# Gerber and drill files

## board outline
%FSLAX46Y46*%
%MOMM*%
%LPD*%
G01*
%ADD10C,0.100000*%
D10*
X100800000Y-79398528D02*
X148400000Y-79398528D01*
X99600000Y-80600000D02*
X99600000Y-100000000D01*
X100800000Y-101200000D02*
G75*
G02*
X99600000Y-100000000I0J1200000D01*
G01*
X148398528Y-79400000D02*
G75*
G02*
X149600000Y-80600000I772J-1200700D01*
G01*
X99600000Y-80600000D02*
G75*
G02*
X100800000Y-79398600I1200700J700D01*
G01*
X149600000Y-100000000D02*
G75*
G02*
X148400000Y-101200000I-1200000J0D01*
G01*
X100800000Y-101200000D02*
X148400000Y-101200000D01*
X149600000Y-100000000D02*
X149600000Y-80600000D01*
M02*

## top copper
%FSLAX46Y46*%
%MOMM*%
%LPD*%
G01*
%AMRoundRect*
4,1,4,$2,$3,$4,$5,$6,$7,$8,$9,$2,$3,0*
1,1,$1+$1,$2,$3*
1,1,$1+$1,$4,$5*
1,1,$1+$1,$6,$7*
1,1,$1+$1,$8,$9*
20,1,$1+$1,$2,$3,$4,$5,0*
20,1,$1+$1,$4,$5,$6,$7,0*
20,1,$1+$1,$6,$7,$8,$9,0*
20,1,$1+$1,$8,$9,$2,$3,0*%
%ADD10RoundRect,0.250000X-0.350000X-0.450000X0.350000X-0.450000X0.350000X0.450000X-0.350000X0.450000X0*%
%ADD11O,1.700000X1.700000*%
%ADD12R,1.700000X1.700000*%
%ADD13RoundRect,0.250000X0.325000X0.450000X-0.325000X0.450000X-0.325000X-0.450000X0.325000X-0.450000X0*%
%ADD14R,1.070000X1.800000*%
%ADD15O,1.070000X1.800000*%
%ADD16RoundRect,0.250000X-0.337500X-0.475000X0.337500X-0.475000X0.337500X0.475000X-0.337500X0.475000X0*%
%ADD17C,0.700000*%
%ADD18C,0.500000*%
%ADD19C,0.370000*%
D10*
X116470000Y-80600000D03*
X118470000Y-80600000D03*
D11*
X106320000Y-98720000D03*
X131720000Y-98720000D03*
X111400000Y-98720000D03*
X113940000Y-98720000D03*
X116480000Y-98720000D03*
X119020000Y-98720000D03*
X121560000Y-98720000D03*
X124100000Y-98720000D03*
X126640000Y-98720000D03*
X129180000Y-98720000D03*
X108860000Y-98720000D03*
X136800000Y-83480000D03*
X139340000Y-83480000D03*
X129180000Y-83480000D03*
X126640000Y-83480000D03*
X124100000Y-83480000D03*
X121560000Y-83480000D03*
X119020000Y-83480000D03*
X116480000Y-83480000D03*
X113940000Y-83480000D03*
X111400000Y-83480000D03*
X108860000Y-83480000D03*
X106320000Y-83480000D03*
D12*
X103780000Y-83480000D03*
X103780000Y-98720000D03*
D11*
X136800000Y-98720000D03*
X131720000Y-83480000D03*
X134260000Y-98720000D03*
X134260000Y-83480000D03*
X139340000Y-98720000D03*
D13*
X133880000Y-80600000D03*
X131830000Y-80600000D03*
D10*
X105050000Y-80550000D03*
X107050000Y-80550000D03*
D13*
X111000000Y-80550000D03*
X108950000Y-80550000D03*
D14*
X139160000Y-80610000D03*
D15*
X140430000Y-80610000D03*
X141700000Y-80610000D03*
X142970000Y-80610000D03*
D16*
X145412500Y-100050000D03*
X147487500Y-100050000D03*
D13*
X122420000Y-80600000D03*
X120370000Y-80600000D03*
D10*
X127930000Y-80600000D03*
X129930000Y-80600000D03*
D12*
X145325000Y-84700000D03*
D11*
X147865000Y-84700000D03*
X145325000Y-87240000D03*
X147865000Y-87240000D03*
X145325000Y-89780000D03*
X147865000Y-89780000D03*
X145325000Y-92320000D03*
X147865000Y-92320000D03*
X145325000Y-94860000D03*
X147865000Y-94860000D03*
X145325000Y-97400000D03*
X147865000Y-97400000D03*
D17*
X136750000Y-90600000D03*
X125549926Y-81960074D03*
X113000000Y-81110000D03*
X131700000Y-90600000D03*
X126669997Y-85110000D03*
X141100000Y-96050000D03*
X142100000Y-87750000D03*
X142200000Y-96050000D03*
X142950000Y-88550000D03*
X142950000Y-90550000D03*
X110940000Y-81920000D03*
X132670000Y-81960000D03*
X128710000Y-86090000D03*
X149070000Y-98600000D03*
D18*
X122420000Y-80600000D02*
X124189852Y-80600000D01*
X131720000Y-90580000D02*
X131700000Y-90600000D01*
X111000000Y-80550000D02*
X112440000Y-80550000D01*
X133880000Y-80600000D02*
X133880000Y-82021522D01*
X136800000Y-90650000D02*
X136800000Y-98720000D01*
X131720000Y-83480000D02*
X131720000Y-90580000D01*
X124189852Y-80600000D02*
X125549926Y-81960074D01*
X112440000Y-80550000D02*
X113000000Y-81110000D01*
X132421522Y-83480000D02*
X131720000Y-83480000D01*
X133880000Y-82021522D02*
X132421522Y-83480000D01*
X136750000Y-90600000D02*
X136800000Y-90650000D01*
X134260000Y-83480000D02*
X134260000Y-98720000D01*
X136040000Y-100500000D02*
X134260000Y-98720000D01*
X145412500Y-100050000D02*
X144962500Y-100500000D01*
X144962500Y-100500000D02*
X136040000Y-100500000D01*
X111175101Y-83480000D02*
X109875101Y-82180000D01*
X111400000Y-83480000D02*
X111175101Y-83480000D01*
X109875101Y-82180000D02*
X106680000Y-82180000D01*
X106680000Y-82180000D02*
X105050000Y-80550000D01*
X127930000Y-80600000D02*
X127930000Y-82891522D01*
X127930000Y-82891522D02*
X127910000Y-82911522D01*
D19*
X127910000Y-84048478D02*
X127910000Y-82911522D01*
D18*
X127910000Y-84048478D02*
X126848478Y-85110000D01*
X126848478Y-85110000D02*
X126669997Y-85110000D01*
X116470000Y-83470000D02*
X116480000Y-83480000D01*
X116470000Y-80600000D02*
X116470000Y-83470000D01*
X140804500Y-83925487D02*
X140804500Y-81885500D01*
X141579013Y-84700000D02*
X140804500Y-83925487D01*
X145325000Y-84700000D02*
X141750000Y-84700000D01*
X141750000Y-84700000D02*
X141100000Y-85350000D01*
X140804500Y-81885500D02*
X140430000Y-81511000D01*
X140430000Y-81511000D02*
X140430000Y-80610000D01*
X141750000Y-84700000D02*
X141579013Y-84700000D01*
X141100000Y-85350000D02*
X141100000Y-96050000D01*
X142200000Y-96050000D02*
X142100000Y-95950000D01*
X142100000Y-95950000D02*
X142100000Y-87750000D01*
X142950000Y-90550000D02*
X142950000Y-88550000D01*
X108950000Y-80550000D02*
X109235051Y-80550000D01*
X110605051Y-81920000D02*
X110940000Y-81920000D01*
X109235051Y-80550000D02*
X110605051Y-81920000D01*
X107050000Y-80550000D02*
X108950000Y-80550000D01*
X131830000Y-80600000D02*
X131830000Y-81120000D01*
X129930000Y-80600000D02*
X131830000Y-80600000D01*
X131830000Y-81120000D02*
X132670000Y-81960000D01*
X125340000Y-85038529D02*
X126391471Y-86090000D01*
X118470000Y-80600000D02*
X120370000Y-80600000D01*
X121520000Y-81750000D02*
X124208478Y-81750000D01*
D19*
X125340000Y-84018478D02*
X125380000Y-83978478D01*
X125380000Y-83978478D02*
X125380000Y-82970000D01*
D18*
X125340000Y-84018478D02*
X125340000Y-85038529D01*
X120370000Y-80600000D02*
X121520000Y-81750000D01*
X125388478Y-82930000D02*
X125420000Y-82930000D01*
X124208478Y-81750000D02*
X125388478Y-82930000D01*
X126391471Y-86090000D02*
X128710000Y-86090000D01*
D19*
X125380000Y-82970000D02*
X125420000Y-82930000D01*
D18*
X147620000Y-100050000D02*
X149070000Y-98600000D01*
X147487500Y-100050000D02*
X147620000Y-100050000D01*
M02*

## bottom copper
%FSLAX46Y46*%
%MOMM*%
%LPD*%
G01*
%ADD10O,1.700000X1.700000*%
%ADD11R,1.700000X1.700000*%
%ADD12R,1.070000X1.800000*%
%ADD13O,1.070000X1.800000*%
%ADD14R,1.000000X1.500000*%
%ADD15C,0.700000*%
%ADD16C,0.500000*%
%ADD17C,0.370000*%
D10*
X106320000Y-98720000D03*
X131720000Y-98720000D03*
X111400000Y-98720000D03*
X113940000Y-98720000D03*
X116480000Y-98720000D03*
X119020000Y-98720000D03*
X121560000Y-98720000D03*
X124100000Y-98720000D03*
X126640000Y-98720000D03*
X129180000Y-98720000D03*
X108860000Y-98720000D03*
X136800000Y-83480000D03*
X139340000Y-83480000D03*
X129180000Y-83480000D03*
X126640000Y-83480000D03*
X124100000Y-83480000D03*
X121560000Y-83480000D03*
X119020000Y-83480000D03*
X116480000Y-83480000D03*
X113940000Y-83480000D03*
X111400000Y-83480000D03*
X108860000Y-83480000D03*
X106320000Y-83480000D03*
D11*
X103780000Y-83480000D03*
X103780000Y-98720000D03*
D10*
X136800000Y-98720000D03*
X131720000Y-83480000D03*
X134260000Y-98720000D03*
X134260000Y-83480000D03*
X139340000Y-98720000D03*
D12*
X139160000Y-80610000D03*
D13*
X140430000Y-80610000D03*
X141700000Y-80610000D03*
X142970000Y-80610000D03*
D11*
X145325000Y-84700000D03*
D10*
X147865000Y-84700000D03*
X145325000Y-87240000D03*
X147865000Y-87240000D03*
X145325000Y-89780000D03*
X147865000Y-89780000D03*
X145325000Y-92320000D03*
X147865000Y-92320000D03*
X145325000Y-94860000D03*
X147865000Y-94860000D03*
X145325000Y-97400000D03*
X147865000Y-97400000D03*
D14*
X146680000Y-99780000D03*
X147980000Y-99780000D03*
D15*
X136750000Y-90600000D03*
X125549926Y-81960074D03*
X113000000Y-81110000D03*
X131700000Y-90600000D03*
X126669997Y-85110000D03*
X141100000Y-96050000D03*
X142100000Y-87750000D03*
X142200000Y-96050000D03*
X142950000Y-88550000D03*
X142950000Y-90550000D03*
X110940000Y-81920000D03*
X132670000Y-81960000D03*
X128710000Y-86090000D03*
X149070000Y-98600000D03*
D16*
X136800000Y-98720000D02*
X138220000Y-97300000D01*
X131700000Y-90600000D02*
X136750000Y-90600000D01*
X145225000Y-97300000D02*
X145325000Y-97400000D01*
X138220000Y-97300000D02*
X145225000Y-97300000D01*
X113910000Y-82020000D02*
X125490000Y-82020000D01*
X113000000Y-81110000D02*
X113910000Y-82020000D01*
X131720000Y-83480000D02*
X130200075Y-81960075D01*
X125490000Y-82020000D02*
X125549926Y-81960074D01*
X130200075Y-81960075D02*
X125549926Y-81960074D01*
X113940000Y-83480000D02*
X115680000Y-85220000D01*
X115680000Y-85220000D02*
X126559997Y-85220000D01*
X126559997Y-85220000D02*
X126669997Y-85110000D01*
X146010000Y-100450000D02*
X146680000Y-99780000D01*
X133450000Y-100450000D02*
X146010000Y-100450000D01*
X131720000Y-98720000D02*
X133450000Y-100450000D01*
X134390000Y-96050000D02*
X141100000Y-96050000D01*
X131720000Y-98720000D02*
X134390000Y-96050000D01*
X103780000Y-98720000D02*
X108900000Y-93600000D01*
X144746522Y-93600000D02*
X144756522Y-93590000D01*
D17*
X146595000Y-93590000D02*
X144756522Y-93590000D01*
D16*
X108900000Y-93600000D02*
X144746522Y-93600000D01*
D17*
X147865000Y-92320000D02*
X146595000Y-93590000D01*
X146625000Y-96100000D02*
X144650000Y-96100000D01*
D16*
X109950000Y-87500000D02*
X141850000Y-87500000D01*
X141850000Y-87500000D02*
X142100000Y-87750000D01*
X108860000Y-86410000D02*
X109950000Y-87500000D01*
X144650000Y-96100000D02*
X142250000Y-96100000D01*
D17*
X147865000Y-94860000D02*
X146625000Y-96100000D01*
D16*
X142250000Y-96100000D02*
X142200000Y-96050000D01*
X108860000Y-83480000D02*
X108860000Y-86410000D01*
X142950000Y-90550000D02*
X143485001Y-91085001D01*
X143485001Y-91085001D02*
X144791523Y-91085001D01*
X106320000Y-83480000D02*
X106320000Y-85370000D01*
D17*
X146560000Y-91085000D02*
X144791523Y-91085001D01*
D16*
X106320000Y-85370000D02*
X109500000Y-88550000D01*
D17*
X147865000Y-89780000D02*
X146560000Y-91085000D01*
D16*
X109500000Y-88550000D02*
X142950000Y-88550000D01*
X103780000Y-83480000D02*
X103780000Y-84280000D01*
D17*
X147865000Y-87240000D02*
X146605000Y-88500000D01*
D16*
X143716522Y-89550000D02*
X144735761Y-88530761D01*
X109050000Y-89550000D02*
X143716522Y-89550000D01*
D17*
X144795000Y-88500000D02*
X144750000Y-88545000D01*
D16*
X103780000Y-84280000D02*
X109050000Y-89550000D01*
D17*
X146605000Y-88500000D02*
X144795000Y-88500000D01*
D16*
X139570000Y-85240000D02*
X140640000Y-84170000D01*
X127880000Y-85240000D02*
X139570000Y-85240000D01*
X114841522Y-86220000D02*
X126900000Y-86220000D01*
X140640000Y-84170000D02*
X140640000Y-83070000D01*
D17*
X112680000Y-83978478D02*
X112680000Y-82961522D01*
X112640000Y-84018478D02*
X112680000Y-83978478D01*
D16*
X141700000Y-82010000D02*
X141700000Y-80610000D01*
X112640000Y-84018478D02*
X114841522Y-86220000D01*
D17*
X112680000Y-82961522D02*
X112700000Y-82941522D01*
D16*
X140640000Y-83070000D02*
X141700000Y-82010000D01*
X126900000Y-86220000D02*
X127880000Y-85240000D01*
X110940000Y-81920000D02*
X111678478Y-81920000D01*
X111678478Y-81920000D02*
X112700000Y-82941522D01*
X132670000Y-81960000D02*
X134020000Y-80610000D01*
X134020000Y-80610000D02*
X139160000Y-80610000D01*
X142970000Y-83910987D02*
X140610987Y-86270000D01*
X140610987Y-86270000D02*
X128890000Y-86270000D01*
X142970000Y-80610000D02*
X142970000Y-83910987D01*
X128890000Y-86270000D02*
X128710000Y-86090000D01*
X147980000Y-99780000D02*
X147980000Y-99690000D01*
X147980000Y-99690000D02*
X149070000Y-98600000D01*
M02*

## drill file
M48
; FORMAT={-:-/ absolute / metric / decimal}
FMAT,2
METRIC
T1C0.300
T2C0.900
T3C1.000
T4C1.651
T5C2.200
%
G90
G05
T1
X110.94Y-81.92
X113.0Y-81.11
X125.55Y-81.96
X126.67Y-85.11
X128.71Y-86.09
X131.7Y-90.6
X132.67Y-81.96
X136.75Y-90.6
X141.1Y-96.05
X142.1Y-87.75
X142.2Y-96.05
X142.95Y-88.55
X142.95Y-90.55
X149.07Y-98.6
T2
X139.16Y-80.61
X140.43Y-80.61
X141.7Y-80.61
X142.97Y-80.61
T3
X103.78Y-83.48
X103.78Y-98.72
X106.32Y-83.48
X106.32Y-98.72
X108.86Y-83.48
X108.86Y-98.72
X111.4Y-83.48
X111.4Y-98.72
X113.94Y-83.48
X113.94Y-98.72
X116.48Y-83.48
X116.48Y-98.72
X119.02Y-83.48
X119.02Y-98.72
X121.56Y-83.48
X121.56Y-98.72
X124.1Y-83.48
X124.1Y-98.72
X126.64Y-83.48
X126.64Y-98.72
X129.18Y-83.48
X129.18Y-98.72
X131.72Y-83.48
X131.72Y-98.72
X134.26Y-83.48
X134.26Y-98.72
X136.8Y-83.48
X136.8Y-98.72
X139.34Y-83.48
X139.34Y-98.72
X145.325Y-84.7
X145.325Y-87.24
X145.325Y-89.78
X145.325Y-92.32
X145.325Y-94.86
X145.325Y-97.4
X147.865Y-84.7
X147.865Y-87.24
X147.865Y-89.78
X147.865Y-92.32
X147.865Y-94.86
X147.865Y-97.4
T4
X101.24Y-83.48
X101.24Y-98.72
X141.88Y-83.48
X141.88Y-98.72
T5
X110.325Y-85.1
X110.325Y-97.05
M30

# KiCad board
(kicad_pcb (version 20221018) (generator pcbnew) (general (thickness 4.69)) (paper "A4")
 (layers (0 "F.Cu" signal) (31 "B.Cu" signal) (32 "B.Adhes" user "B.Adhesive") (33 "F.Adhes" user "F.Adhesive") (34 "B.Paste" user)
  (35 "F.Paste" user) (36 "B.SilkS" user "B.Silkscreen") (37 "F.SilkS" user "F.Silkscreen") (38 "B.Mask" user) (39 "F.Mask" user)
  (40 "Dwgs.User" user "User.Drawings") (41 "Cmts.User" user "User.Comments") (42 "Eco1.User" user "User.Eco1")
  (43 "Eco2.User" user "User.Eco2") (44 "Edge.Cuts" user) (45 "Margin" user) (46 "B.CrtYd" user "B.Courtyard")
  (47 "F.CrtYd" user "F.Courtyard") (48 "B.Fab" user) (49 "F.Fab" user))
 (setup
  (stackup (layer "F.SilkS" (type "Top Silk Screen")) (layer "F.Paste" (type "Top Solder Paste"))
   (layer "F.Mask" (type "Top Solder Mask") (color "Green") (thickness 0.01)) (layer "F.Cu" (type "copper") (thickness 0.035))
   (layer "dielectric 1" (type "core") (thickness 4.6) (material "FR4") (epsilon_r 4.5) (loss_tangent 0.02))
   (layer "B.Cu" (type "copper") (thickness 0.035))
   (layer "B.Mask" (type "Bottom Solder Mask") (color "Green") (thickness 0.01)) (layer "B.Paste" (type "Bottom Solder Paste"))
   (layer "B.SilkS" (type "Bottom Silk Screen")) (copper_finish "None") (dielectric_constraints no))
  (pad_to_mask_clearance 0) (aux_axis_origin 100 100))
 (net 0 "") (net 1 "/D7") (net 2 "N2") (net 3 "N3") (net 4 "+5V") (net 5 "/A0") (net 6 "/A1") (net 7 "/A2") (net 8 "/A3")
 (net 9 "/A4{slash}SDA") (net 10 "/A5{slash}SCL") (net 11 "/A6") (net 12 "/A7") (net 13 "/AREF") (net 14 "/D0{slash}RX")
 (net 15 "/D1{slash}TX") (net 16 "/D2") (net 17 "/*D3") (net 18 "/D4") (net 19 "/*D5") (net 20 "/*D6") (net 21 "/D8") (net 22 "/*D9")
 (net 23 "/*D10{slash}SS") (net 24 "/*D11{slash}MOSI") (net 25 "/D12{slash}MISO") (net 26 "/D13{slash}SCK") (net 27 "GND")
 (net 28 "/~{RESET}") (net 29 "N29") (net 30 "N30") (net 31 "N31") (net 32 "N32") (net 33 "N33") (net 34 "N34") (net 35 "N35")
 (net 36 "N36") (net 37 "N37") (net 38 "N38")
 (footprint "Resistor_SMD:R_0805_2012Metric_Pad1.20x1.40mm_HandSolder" (layer "F.Cu") (at 117.47 80.6)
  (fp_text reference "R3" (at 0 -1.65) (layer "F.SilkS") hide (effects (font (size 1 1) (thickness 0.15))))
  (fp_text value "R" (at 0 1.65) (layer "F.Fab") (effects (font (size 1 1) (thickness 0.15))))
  (pad "1" smd roundrect (at -1 0) (size 1.2 1.4) (layers "F.Cu" "F.Paste" "F.Mask") (roundrect_rratio 0.208333) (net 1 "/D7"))
  (pad "2" smd roundrect (at 1 0) (size 1.2 1.4) (layers "F.Cu" "F.Paste" "F.Mask") (roundrect_rratio 0.208333) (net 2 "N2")))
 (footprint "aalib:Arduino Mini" (layer "F.Cu") (at 121.56 91.1 90)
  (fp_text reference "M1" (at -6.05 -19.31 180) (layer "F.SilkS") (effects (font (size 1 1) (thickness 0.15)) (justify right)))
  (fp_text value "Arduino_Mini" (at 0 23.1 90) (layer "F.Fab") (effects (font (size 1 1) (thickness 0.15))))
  (pad "" np_thru_hole circle (at -7.62 -20.32 90) (size 1.651 1.651) (drill 1.651) (layers "*.Mask"))
  (pad "" np_thru_hole circle (at -7.62 20.32 90) (size 1.651 1.651) (drill 1.651) (layers "*.Mask"))
  (pad "" np_thru_hole circle (at 7.62 -20.32 90) (size 1.651 1.651) (drill 1.651) (layers "*.Mask"))
  (pad "" np_thru_hole circle (at 7.62 20.32 90) (size 1.651 1.651) (drill 1.651) (layers "*.Mask"))
  (pad "3V3" thru_hole oval (at -7.62 -15.24 90) (size 1.7 1.7) (drill 1) (layers "*.Cu" "*.Mask") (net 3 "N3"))
  (pad "5V" thru_hole oval (at -7.62 10.16 90) (size 1.7 1.7) (drill 1) (layers "*.Cu" "*.Mask") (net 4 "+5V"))
  (pad "A0" thru_hole oval (at -7.62 -10.16 90) (size 1.7 1.7) (drill 1) (layers "*.Cu" "*.Mask") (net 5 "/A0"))
  (pad "A1" thru_hole oval (at -7.62 -7.62 90) (size 1.7 1.7) (drill 1) (layers "*.Cu" "*.Mask") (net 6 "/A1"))
  (pad "A2" thru_hole oval (at -7.62 -5.08 90) (size 1.7 1.7) (drill 1) (layers "*.Cu" "*.Mask") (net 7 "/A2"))
  (pad "A3" thru_hole oval (at -7.62 -2.54 90) (size 1.7 1.7) (drill 1) (layers "*.Cu" "*.Mask") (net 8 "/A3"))
  (pad "A4" thru_hole oval (at -7.62 0 90) (size 1.7 1.7) (drill 1) (layers "*.Cu" "*.Mask") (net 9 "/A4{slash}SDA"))
  (pad "A5" thru_hole oval (at -7.62 2.54 90) (size 1.7 1.7) (drill 1) (layers "*.Cu" "*.Mask") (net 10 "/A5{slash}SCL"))
  (pad "A6" thru_hole oval (at -7.62 5.08 90) (size 1.7 1.7) (drill 1) (layers "*.Cu" "*.Mask") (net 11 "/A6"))
  (pad "A7" thru_hole oval (at -7.62 7.62 90) (size 1.7 1.7) (drill 1) (layers "*.Cu" "*.Mask") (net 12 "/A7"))
  (pad "AREF" thru_hole oval (at -7.62 -12.7 90) (size 1.7 1.7) (drill 1) (layers "*.Cu" "*.Mask") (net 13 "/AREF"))
  (pad "D0/RX" thru_hole oval (at 7.62 15.24 90) (size 1.7 1.7) (drill 1) (layers "*.Cu" "*.Mask") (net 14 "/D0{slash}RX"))
  (pad "D1/TX" thru_hole oval (at 7.62 17.78 90) (size 1.7 1.7) (drill 1) (layers "*.Cu" "*.Mask") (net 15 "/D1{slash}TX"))
  (pad "D2" thru_hole oval (at 7.62 7.62 90) (size 1.7 1.7) (drill 1) (layers "*.Cu" "*.Mask") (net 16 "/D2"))
  (pad "D3" thru_hole oval (at 7.62 5.08 90) (size 1.7 1.7) (drill 1) (layers "*.Cu" "*.Mask") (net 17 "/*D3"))
  (pad "D4" thru_hole oval (at 7.62 2.54 90) (size 1.7 1.7) (drill 1) (layers "*.Cu" "*.Mask") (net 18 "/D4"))
  (pad "D5" thru_hole oval (at 7.62 0 90) (size 1.7 1.7) (drill 1) (layers "*.Cu" "*.Mask") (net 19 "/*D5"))
  (pad "D6" thru_hole oval (at 7.62 -2.54 90) (size 1.7 1.7) (drill 1) (layers "*.Cu" "*.Mask") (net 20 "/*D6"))
  (pad "D7" thru_hole oval (at 7.62 -5.08 90) (size 1.7 1.7) (drill 1) (layers "*.Cu" "*.Mask") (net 1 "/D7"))
  (pad "D8" thru_hole oval (at 7.62 -7.62 90) (size 1.7 1.7) (drill 1) (layers "*.Cu" "*.Mask") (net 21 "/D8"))
  (pad "D9" thru_hole oval (at 7.62 -10.16 90) (size 1.7 1.7) (drill 1) (layers "*.Cu" "*.Mask") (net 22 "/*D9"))
  (pad "D10" thru_hole oval (at 7.62 -12.7 90) (size 1.7 1.7) (drill 1) (layers "*.Cu" "*.Mask") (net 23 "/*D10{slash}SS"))
  (pad "D11" thru_hole oval (at 7.62 -15.24 90) (size 1.7 1.7) (drill 1) (layers "*.Cu" "*.Mask") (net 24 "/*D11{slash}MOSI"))
  (pad "D12" thru_hole rect (at 7.62 -17.78 90) (size 1.7 1.7) (drill 1) (layers "*.Cu" "*.Mask") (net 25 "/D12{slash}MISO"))
  (pad "D13" thru_hole rect (at -7.62 -17.78 90) (size 1.7 1.7) (drill 1) (layers "*.Cu" "*.Mask") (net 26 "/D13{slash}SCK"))
  (pad "GND" thru_hole oval (at -7.62 15.24 90) (size 1.7 1.7) (drill 1) (layers "*.Cu" "*.Mask") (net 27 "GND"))
  (pad "GND" thru_hole oval (at 7.62 10.16 90) (size 1.7 1.7) (drill 1) (layers "*.Cu" "*.Mask") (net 27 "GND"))
  (pad "RESET" thru_hole oval (at -7.62 12.7 90) (size 1.7 1.7) (drill 1) (layers "*.Cu" "*.Mask") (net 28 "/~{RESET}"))
  (pad "RESET" thru_hole oval (at 7.62 12.7 90) (size 1.7 1.7) (drill 1) (layers "*.Cu" "*.Mask") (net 28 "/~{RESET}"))
  (pad "VIN" thru_hole oval (at -7.62 17.78 90) (size 1.7 1.7) (drill 1) (layers "*.Cu" "*.Mask") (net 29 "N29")))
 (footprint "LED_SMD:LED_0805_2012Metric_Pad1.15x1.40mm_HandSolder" (layer "F.Cu") (at 132.855 80.6 180)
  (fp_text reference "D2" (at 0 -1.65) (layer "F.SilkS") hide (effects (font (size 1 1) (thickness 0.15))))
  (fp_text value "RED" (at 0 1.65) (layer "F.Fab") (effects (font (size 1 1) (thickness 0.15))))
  (pad "1" smd roundrect (at -1.025 0 180) (size 1.15 1.4) (layers "F.Cu" "F.Paste" "F.Mask") (roundrect_rratio 0.2173913043) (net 27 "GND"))
  (pad "2" smd roundrect (at 1.025 0 180) (size 1.15 1.4) (layers "F.Cu" "F.Paste" "F.Mask") (roundrect_rratio 0.2173913043) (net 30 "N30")))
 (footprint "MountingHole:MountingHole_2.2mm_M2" (layer "F.Cu") (at 110.325 85.1)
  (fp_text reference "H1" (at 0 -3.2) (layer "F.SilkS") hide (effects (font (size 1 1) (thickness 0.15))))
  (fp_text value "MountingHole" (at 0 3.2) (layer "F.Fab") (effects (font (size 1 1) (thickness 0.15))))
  (pad "" np_thru_hole circle (at 0 0) (size 2.2 2.2) (drill 2.2) (layers "*.Cu" "*.Mask")))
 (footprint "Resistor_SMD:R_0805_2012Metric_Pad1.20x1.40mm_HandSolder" (layer "F.Cu") (at 106.05 80.55)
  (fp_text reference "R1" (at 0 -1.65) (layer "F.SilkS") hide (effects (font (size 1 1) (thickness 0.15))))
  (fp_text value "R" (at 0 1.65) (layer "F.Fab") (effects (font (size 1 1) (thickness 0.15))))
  (pad "1" smd roundrect (at -1 0) (size 1.2 1.4) (layers "F.Cu" "F.Paste" "F.Mask") (roundrect_rratio 0.208333) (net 22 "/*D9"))
  (pad "2" smd roundrect (at 1 0) (size 1.2 1.4) (layers "F.Cu" "F.Paste" "F.Mask") (roundrect_rratio 0.208333) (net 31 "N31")))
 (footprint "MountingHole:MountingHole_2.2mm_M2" (layer "F.Cu") (at 110.325 97.05)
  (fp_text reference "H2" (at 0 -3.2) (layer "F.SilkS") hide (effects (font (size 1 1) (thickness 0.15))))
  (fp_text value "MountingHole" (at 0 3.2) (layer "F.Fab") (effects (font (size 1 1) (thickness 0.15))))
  (pad "" np_thru_hole circle (at 0 0) (size 2.2 2.2) (drill 2.2) (layers "*.Cu" "*.Mask")))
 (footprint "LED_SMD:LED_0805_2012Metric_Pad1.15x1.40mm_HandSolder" (layer "F.Cu") (at 109.975 80.55 180)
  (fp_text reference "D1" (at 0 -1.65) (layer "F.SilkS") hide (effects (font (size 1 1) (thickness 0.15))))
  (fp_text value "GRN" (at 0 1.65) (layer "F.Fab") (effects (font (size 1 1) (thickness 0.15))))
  (pad "1" smd roundrect (at -1.025 0 180) (size 1.15 1.4) (layers "F.Cu" "F.Paste" "F.Mask") (roundrect_rratio 0.2173913043) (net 27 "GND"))
  (pad "2" smd roundrect (at 1.025 0 180) (size 1.15 1.4) (layers "F.Cu" "F.Paste" "F.Mask") (roundrect_rratio 0.2173913043) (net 31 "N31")))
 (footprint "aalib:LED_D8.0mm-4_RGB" (layer "F.Cu") (at 139.16 80.61)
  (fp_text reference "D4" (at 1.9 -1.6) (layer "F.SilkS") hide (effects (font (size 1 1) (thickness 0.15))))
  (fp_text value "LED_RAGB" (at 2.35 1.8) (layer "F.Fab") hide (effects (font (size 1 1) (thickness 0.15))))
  (pad "1" thru_hole rect (at 0 0) (size 1.07 1.8) (drill 0.9) (layers "*.Cu" "*.Mask") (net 30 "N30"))
  (pad "2" thru_hole oval (at 1.27 0) (size 1.07 1.8) (drill 0.9) (layers "*.Cu" "*.Mask") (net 4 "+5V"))
  (pad "3" thru_hole oval (at 2.54 0) (size 1.07 1.8) (drill 0.9) (layers "*.Cu" "*.Mask") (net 31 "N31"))
  (pad "4" thru_hole oval (at 3.81 0) (size 1.07 1.8) (drill 0.9) (layers "*.Cu" "*.Mask") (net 2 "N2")))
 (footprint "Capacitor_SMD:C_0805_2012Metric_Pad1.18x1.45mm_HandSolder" (layer "F.Cu") (at 146.45 100.05)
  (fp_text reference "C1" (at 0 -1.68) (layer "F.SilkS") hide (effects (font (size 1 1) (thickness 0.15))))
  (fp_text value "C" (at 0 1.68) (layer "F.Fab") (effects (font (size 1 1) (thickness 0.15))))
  (pad "1" smd roundrect (at -1.0375 0) (size 1.175 1.45) (layers "F.Cu" "F.Paste" "F.Mask") (roundrect_rratio 0.2127659574)
   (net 28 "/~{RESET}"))
  (pad "2" smd roundrect (at 1.0375 0) (size 1.175 1.45) (layers "F.Cu" "F.Paste" "F.Mask") (roundrect_rratio 0.2127659574) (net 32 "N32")))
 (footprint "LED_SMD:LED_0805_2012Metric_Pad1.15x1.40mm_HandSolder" (layer "F.Cu") (at 121.395 80.6 180)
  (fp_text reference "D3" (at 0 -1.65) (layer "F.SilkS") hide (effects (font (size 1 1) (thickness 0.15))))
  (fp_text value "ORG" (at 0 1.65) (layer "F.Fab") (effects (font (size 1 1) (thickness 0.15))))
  (pad "1" smd roundrect (at -1.025 0 180) (size 1.15 1.4) (layers "F.Cu" "F.Paste" "F.Mask") (roundrect_rratio 0.2173913043) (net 27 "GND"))
  (pad "2" smd roundrect (at 1.025 0 180) (size 1.15 1.4) (layers "F.Cu" "F.Paste" "F.Mask") (roundrect_rratio 0.2173913043) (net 2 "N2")))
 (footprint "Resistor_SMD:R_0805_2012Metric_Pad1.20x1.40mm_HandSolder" (layer "F.Cu") (at 128.93 80.6)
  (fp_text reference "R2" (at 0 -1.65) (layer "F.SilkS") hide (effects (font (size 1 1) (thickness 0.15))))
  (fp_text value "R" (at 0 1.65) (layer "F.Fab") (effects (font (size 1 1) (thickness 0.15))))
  (pad "1" smd roundrect (at -1 0) (size 1.2 1.4) (layers "F.Cu" "F.Paste" "F.Mask") (roundrect_rratio 0.208333) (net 21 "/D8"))
  (pad "2" smd roundrect (at 1 0) (size 1.2 1.4) (layers "F.Cu" "F.Paste" "F.Mask") (roundrect_rratio 0.208333) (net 30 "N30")))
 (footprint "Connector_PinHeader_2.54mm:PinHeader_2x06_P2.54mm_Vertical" (layer "F.Cu") (at 145.325 84.7)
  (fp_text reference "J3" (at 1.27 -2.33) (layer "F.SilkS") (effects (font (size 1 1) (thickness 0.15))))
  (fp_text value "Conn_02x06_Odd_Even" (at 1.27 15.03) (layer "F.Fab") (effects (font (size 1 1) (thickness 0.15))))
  (pad "1" thru_hole rect (at 0 0) (size 1.7 1.7) (drill 1) (layers "*.Cu" "*.Mask") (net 4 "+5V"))
  (pad "2" thru_hole oval (at 2.54 0) (size 1.7 1.7) (drill 1) (layers "*.Cu" "*.Mask") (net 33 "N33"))
  (pad "3" thru_hole oval (at 0 2.54) (size 1.7 1.7) (drill 1) (layers "*.Cu" "*.Mask") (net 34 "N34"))
  (pad "4" thru_hole oval (at 2.54 2.54) (size 1.7 1.7) (drill 1) (layers "*.Cu" "*.Mask") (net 25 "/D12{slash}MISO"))
  (pad "5" thru_hole oval (at 0 5.08) (size 1.7 1.7) (drill 1) (layers "*.Cu" "*.Mask") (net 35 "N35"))
  (pad "6" thru_hole oval (at 2.54 5.08) (size 1.7 1.7) (drill 1) (layers "*.Cu" "*.Mask") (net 24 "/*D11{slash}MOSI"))
  (pad "7" thru_hole oval (at 0 7.62) (size 1.7 1.7) (drill 1) (layers "*.Cu" "*.Mask") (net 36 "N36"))
  (pad "8" thru_hole oval (at 2.54 7.62) (size 1.7 1.7) (drill 1) (layers "*.Cu" "*.Mask") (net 26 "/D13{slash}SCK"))
  (pad "9" thru_hole oval (at 0 10.16) (size 1.7 1.7) (drill 1) (layers "*.Cu" "*.Mask") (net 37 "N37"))
  (pad "10" thru_hole oval (at 2.54 10.16) (size 1.7 1.7) (drill 1) (layers "*.Cu" "*.Mask") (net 23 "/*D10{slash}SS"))
  (pad "11" thru_hole oval (at 0 12.7) (size 1.7 1.7) (drill 1) (layers "*.Cu" "*.Mask") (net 27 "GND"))
  (pad "12" thru_hole oval (at 2.54 12.7) (size 1.7 1.7) (drill 1) (layers "*.Cu" "*.Mask") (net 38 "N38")))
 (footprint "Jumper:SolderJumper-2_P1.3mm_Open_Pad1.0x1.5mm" (layer "B.Cu") (at 147.33 99.78)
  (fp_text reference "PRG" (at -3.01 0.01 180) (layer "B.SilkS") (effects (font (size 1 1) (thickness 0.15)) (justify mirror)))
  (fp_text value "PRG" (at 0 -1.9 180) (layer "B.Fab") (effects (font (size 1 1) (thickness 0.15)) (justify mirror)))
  (pad "1" smd rect (at -0.65 0) (size 1 1.5) (layers "B.Cu" "B.Mask") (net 4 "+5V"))
  (pad "2" smd rect (at 0.65 0) (size 1 1.5) (layers "B.Cu" "B.Mask") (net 32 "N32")))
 (gr_line (start 100.8 79.398528) (end 148.4 79.398528) (stroke (width 0.1) (type solid)) (layer "Edge.Cuts"))
 (gr_line (start 99.6 80.6) (end 99.6 100) (stroke (width 0.1) (type solid)) (layer "Edge.Cuts"))
 (gr_arc (start 100.8 101.2) (mid 99.951472 100.848528) (end 99.6 100) (stroke (width 0.1) (type default)) (layer "Edge.Cuts"))
 (gr_arc (start 148.398528 79.4) (mid 149.247791 79.751167) (end 149.6 80.6) (stroke (width 0.1) (type default)) (layer "Edge.Cuts"))
 (gr_arc (start 99.6 80.6) (mid 99.951163 79.750732) (end 100.8 79.398528) (stroke (width 0.1) (type default)) (layer "Edge.Cuts"))
 (gr_arc (start 149.6 100) (mid 149.248524 100.848524) (end 148.4 101.2) (stroke (width 0.1) (type default)) (layer "Edge.Cuts"))
 (gr_line (start 100.8 101.2) (end 148.4 101.2) (stroke (width 0.1) (type solid)) (layer "Edge.Cuts"))
 (gr_line (start 149.6 100) (end 149.6 80.6) (stroke (width 0.1) (type solid)) (layer "Edge.Cuts"))
 (segment (start 122.42 80.6) (end 124.189852 80.6) (width 0.5) (layer "F.Cu") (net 27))
 (segment (start 131.72 90.58) (end 131.7 90.6) (width 0.5) (layer "F.Cu") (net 27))
 (segment (start 111 80.55) (end 112.44 80.55) (width 0.5) (layer "F.Cu") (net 27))
 (segment (start 133.88 80.6) (end 133.88 82.021522) (width 0.5) (layer "F.Cu") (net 27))
 (segment (start 136.8 90.65) (end 136.8 98.72) (width 0.5) (layer "F.Cu") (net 27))
 (segment (start 131.72 83.48) (end 131.72 90.58) (width 0.5) (layer "F.Cu") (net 27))
 (segment (start 124.189852 80.6) (end 125.549926 81.960074) (width 0.5) (layer "F.Cu") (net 27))
 (segment (start 112.44 80.55) (end 113 81.11) (width 0.5) (layer "F.Cu") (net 27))
 (segment (start 132.421522 83.48) (end 131.72 83.48) (width 0.5) (layer "F.Cu") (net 27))
 (segment (start 133.88 82.021522) (end 132.421522 83.48) (width 0.5) (layer "F.Cu") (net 27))
 (segment (start 136.75 90.6) (end 136.8 90.65) (width 0.5) (layer "F.Cu") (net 27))
 (via (at 136.75 90.6) (size 0.7) (drill 0.3) (layers "F.Cu" "B.Cu") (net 27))
 (via (at 125.549926 81.960074) (size 0.7) (drill 0.3) (layers "F.Cu" "B.Cu") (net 27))
 (via (at 113 81.11) (size 0.7) (drill 0.3) (layers "F.Cu" "B.Cu") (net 27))
 (via (at 131.7 90.6) (size 0.7) (drill 0.3) (layers "F.Cu" "B.Cu") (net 27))
 (segment (start 136.8 98.72) (end 138.22 97.3) (width 0.5) (layer "B.Cu") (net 27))
 (segment (start 131.7 90.6) (end 136.75 90.6) (width 0.5) (layer "B.Cu") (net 27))
 (segment (start 145.225 97.3) (end 145.325 97.4) (width 0.5) (layer "B.Cu") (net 27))
 (segment (start 138.22 97.3) (end 145.225 97.3) (width 0.5) (layer "B.Cu") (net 27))
 (segment (start 113.91 82.02) (end 125.49 82.02) (width 0.5) (layer "B.Cu") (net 27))
 (segment (start 113 81.11) (end 113.91 82.02) (width 0.5) (layer "B.Cu") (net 27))
 (segment (start 131.72 83.48) (end 130.200075 81.960075) (width 0.5) (layer "B.Cu") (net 27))
 (segment (start 125.49 82.02) (end 125.549926 81.960074) (width 0.5) (layer "B.Cu") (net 27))
 (segment (start 130.200075 81.960075) (end 125.549926 81.960074) (width 0.5) (layer "B.Cu") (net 27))
 (segment (start 134.26 83.48) (end 134.26 98.72) (width 0.5) (layer "F.Cu") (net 28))
 (segment (start 136.04 100.5) (end 134.26 98.72) (width 0.5) (layer "F.Cu") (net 28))
 (segment (start 145.4125 100.05) (end 144.9625 100.5) (width 0.5) (layer "F.Cu") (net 28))
 (segment (start 144.9625 100.5) (end 136.04 100.5) (width 0.5) (layer "F.Cu") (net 28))
 (segment (start 111.175101 83.48) (end 109.875101 82.18) (width 0.5) (layer "F.Cu") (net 22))
 (segment (start 111.4 83.48) (end 111.175101 83.48) (width 0.5) (layer "F.Cu") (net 22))
 (segment (start 109.875101 82.18) (end 106.68 82.18) (width 0.5) (layer "F.Cu") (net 22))
 (segment (start 106.68 82.18) (end 105.05 80.55) (width 0.5) (layer "F.Cu") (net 22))
 (segment (start 127.93 80.6) (end 127.93 82.891522) (width 0.5) (layer "F.Cu") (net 21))
 (segment (start 127.93 82.891522) (end 127.91 82.911522) (width 0.5) (layer "F.Cu") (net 21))
 (segment (start 127.91 84.048478) (end 127.91 82.911522) (width 0.37) (layer "F.Cu") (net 21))
 (segment (start 127.91 84.048478) (end 126.848478 85.11) (width 0.5) (layer "F.Cu") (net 21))
 (segment (start 126.848478 85.11) (end 126.669997 85.11) (width 0.5) (layer "F.Cu") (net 21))
 (via (at 126.669997 85.11) (size 0.7) (drill 0.3) (layers "F.Cu" "B.Cu") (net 21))
 (segment (start 113.94 83.48) (end 115.68 85.22) (width 0.5) (layer "B.Cu") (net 21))
 (segment (start 115.68 85.22) (end 126.559997 85.22) (width 0.5) (layer "B.Cu") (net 21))
 (segment (start 126.559997 85.22) (end 126.669997 85.11) (width 0.5) (layer "B.Cu") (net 21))
 (segment (start 116.47 83.47) (end 116.48 83.48) (width 0.5) (layer "F.Cu") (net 1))
 (segment (start 116.47 80.6) (end 116.47 83.47) (width 0.5) (layer "F.Cu") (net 1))
 (segment (start 140.8045 83.925487) (end 140.8045 81.8855) (width 0.5) (layer "F.Cu") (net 4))
 (segment (start 141.579013 84.7) (end 140.8045 83.925487) (width 0.5) (layer "F.Cu") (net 4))
 (segment (start 145.325 84.7) (end 141.75 84.7) (width 0.5) (layer "F.Cu") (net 4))
 (segment (start 141.75 84.7) (end 141.1 85.35) (width 0.5) (layer "F.Cu") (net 4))
 (segment (start 140.8045 81.8855) (end 140.43 81.511) (width 0.5) (layer "F.Cu") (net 4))
 (segment (start 140.43 81.511) (end 140.43 80.61) (width 0.5) (layer "F.Cu") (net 4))
 (segment (start 141.75 84.7) (end 141.579013 84.7) (width 0.5) (layer "F.Cu") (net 4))
 (segment (start 141.1 85.35) (end 141.1 96.05) (width 0.5) (layer "F.Cu") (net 4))
 (via (at 141.1 96.05) (size 0.7) (drill 0.3) (layers "F.Cu" "B.Cu") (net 4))
 (segment (start 146.01 100.45) (end 146.68 99.78) (width 0.5) (layer "B.Cu") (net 4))
 (segment (start 133.45 100.45) (end 146.01 100.45) (width 0.5) (layer "B.Cu") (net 4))
 (segment (start 131.72 98.72) (end 133.45 100.45) (width 0.5) (layer "B.Cu") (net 4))
 (segment (start 134.39 96.05) (end 141.1 96.05) (width 0.5) (layer "B.Cu") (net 4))
 (segment (start 131.72 98.72) (end 134.39 96.05) (width 0.5) (layer "B.Cu") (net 4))
 (segment (start 103.78 98.72) (end 108.9 93.6) (width 0.5) (layer "B.Cu") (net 26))
 (segment (start 144.746522 93.6) (end 144.756522 93.59) (width 0.5) (layer "B.Cu") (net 26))
 (segment (start 146.595 93.59) (end 144.756522 93.59) (width 0.37) (layer "B.Cu") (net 26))
 (segment (start 108.9 93.6) (end 144.746522 93.6) (width 0.5) (layer "B.Cu") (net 26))
 (segment (start 147.865 92.32) (end 146.595 93.59) (width 0.37) (layer "B.Cu") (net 26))
 (segment (start 142.2 96.05) (end 142.1 95.95) (width 0.5) (layer "F.Cu") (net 23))
 (segment (start 142.1 95.95) (end 142.1 87.75) (width 0.5) (layer "F.Cu") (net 23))
 (via (at 142.1 87.75) (size 0.7) (drill 0.3) (layers "F.Cu" "B.Cu") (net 23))
 (via (at 142.2 96.05) (size 0.7) (drill 0.3) (layers "F.Cu" "B.Cu") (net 23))
 (segment (start 146.625 96.1) (end 144.65 96.1) (width 0.37) (layer "B.Cu") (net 23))
 (segment (start 109.95 87.5) (end 141.85 87.5) (width 0.5) (layer "B.Cu") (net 23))
 (segment (start 141.85 87.5) (end 142.1 87.75) (width 0.5) (layer "B.Cu") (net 23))
 (segment (start 108.86 86.41) (end 109.95 87.5) (width 0.5) (layer "B.Cu") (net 23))
 (segment (start 144.65 96.1) (end 142.25 96.1) (width 0.5) (layer "B.Cu") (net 23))
 (segment (start 147.865 94.86) (end 146.625 96.1) (width 0.37) (layer "B.Cu") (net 23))
 (segment (start 142.25 96.1) (end 142.2 96.05) (width 0.5) (layer "B.Cu") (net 23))
 (segment (start 108.86 83.48) (end 108.86 86.41) (width 0.5) (layer "B.Cu") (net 23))
 (segment (start 142.95 90.55) (end 142.95 88.55) (width 0.5) (layer "F.Cu") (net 24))
 (via (at 142.95 88.55) (size 0.7) (drill 0.3) (layers "F.Cu" "B.Cu") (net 24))
 (via (at 142.95 90.55) (size 0.7) (drill 0.3) (layers "F.Cu" "B.Cu") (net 24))
 (segment (start 142.95 90.55) (end 143.485001 91.085001) (width 0.5) (layer "B.Cu") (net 24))
 (segment (start 143.485001 91.085001) (end 144.791523 91.085001) (width 0.5) (layer "B.Cu") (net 24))
 (segment (start 106.32 83.48) (end 106.32 85.37) (width 0.5) (layer "B.Cu") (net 24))
 (segment (start 146.56 91.085) (end 144.791523 91.085001) (width 0.37) (layer "B.Cu") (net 24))
 (segment (start 106.32 85.37) (end 109.5 88.55) (width 0.5) (layer "B.Cu") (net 24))
 (segment (start 147.865 89.78) (end 146.56 91.085) (width 0.37) (layer "B.Cu") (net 24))
 (segment (start 109.5 88.55) (end 142.95 88.55) (width 0.5) (layer "B.Cu") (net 24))
 (segment (start 103.78 83.48) (end 103.78 84.28) (width 0.5) (layer "B.Cu") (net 25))
 (segment (start 147.865 87.24) (end 146.605 88.5) (width 0.37) (layer "B.Cu") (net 25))
 (segment (start 143.716522 89.55) (end 144.735761 88.530761) (width 0.5) (layer "B.Cu") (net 25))
 (segment (start 109.05 89.55) (end 143.716522 89.55) (width 0.5) (layer "B.Cu") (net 25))
 (segment (start 144.795 88.5) (end 144.75 88.545) (width 0.37) (layer "B.Cu") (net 25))
 (segment (start 103.78 84.28) (end 109.05 89.55) (width 0.5) (layer "B.Cu") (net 25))
 (segment (start 146.605 88.5) (end 144.795 88.5) (width 0.37) (layer "B.Cu") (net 25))
 (segment (start 108.95 80.55) (end 109.235051 80.55) (width 0.5) (layer "F.Cu") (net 31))
 (segment (start 110.605051 81.92) (end 110.94 81.92) (width 0.5) (layer "F.Cu") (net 31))
 (segment (start 109.235051 80.55) (end 110.605051 81.92) (width 0.5) (layer "F.Cu") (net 31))
 (segment (start 107.05 80.55) (end 108.95 80.55) (width 0.5) (layer "F.Cu") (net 31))
 (via (at 110.94 81.92) (size 0.7) (drill 0.3) (layers "F.Cu" "B.Cu") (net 31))
 (segment (start 139.57 85.24) (end 140.64 84.17) (width 0.5) (layer "B.Cu") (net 31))
 (segment (start 127.88 85.24) (end 139.57 85.24) (width 0.5) (layer "B.Cu") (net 31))
 (segment (start 114.841522 86.22) (end 126.9 86.22) (width 0.5) (layer "B.Cu") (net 31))
 (segment (start 140.64 84.17) (end 140.64 83.07) (width 0.5) (layer "B.Cu") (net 31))
 (segment (start 112.68 83.978478) (end 112.68 82.961522) (width 0.37) (layer "B.Cu") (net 31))
 (segment (start 112.64 84.018478) (end 112.68 83.978478) (width 0.37) (layer "B.Cu") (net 31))
 (segment (start 141.7 82.01) (end 141.7 80.61) (width 0.5) (layer "B.Cu") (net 31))
 (segment (start 112.64 84.018478) (end 114.841522 86.22) (width 0.5) (layer "B.Cu") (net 31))
 (segment (start 112.68 82.961522) (end 112.7 82.941522) (width 0.37) (layer "B.Cu") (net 31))
 (segment (start 140.64 83.07) (end 141.7 82.01) (width 0.5) (layer "B.Cu") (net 31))
 (segment (start 126.9 86.22) (end 127.88 85.24) (width 0.5) (layer "B.Cu") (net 31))
 (segment (start 110.94 81.92) (end 111.678478 81.92) (width 0.5) (layer "B.Cu") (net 31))
 (segment (start 111.678478 81.92) (end 112.7 82.941522) (width 0.5) (layer "B.Cu") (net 31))
 (segment (start 131.83 80.6) (end 131.83 81.12) (width 0.5) (layer "F.Cu") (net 30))
 (segment (start 129.93 80.6) (end 131.83 80.6) (width 0.5) (layer "F.Cu") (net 30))
 (segment (start 131.83 81.12) (end 132.67 81.96) (width 0.5) (layer "F.Cu") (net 30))
 (via (at 132.67 81.96) (size 0.7) (drill 0.3) (layers "F.Cu" "B.Cu") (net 30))
 (segment (start 132.67 81.96) (end 134.02 80.61) (width 0.5) (layer "B.Cu") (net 30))
 (segment (start 134.02 80.61) (end 139.16 80.61) (width 0.5) (layer "B.Cu") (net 30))
 (segment (start 125.34 85.038529) (end 126.391471 86.09) (width 0.5) (layer "F.Cu") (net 2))
 (segment (start 118.47 80.6) (end 120.37 80.6) (width 0.5) (layer "F.Cu") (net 2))
 (segment (start 121.52 81.75) (end 124.208478 81.75) (width 0.5) (layer "F.Cu") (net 2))
 (segment (start 125.34 84.018478) (end 125.38 83.978478) (width 0.37) (layer "F.Cu") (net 2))
 (segment (start 125.38 83.978478) (end 125.38 82.97) (width 0.37) (layer "F.Cu") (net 2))
 (segment (start 125.34 84.018478) (end 125.34 85.038529) (width 0.5) (layer "F.Cu") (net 2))
 (segment (start 120.37 80.6) (end 121.52 81.75) (width 0.5) (layer "F.Cu") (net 2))
 (segment (start 125.388478 82.93) (end 125.42 82.93) (width 0.5) (layer "F.Cu") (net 2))
 (segment (start 124.208478 81.75) (end 125.388478 82.93) (width 0.5) (layer "F.Cu") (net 2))
 (segment (start 126.391471 86.09) (end 128.71 86.09) (width 0.5) (layer "F.Cu") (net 2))
 (segment (start 125.38 82.97) (end 125.42 82.93) (width 0.37) (layer "F.Cu") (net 2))
 (via (at 128.71 86.09) (size 0.7) (drill 0.3) (layers "F.Cu" "B.Cu") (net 2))
 (segment (start 142.97 83.910987) (end 140.610987 86.27) (width 0.5) (layer "B.Cu") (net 2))
 (segment (start 140.610987 86.27) (end 128.89 86.27) (width 0.5) (layer "B.Cu") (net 2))
 (segment (start 142.97 80.61) (end 142.97 83.910987) (width 0.5) (layer "B.Cu") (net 2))
 (segment (start 128.89 86.27) (end 128.71 86.09) (width 0.5) (layer "B.Cu") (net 2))
 (segment (start 147.62 100.05) (end 149.07 98.6) (width 0.5) (layer "F.Cu") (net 32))
 (segment (start 147.4875 100.05) (end 147.62 100.05) (width 0.5) (layer "F.Cu") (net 32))
 (via (at 149.07 98.6) (size 0.7) (drill 0.3) (layers "F.Cu" "B.Cu") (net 32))
 (segment (start 147.98 99.78) (end 147.98 99.69) (width 0.5) (layer "B.Cu") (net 32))
 (segment (start 147.98 99.69) (end 149.07 98.6) (width 0.5) (layer "B.Cu") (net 32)))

